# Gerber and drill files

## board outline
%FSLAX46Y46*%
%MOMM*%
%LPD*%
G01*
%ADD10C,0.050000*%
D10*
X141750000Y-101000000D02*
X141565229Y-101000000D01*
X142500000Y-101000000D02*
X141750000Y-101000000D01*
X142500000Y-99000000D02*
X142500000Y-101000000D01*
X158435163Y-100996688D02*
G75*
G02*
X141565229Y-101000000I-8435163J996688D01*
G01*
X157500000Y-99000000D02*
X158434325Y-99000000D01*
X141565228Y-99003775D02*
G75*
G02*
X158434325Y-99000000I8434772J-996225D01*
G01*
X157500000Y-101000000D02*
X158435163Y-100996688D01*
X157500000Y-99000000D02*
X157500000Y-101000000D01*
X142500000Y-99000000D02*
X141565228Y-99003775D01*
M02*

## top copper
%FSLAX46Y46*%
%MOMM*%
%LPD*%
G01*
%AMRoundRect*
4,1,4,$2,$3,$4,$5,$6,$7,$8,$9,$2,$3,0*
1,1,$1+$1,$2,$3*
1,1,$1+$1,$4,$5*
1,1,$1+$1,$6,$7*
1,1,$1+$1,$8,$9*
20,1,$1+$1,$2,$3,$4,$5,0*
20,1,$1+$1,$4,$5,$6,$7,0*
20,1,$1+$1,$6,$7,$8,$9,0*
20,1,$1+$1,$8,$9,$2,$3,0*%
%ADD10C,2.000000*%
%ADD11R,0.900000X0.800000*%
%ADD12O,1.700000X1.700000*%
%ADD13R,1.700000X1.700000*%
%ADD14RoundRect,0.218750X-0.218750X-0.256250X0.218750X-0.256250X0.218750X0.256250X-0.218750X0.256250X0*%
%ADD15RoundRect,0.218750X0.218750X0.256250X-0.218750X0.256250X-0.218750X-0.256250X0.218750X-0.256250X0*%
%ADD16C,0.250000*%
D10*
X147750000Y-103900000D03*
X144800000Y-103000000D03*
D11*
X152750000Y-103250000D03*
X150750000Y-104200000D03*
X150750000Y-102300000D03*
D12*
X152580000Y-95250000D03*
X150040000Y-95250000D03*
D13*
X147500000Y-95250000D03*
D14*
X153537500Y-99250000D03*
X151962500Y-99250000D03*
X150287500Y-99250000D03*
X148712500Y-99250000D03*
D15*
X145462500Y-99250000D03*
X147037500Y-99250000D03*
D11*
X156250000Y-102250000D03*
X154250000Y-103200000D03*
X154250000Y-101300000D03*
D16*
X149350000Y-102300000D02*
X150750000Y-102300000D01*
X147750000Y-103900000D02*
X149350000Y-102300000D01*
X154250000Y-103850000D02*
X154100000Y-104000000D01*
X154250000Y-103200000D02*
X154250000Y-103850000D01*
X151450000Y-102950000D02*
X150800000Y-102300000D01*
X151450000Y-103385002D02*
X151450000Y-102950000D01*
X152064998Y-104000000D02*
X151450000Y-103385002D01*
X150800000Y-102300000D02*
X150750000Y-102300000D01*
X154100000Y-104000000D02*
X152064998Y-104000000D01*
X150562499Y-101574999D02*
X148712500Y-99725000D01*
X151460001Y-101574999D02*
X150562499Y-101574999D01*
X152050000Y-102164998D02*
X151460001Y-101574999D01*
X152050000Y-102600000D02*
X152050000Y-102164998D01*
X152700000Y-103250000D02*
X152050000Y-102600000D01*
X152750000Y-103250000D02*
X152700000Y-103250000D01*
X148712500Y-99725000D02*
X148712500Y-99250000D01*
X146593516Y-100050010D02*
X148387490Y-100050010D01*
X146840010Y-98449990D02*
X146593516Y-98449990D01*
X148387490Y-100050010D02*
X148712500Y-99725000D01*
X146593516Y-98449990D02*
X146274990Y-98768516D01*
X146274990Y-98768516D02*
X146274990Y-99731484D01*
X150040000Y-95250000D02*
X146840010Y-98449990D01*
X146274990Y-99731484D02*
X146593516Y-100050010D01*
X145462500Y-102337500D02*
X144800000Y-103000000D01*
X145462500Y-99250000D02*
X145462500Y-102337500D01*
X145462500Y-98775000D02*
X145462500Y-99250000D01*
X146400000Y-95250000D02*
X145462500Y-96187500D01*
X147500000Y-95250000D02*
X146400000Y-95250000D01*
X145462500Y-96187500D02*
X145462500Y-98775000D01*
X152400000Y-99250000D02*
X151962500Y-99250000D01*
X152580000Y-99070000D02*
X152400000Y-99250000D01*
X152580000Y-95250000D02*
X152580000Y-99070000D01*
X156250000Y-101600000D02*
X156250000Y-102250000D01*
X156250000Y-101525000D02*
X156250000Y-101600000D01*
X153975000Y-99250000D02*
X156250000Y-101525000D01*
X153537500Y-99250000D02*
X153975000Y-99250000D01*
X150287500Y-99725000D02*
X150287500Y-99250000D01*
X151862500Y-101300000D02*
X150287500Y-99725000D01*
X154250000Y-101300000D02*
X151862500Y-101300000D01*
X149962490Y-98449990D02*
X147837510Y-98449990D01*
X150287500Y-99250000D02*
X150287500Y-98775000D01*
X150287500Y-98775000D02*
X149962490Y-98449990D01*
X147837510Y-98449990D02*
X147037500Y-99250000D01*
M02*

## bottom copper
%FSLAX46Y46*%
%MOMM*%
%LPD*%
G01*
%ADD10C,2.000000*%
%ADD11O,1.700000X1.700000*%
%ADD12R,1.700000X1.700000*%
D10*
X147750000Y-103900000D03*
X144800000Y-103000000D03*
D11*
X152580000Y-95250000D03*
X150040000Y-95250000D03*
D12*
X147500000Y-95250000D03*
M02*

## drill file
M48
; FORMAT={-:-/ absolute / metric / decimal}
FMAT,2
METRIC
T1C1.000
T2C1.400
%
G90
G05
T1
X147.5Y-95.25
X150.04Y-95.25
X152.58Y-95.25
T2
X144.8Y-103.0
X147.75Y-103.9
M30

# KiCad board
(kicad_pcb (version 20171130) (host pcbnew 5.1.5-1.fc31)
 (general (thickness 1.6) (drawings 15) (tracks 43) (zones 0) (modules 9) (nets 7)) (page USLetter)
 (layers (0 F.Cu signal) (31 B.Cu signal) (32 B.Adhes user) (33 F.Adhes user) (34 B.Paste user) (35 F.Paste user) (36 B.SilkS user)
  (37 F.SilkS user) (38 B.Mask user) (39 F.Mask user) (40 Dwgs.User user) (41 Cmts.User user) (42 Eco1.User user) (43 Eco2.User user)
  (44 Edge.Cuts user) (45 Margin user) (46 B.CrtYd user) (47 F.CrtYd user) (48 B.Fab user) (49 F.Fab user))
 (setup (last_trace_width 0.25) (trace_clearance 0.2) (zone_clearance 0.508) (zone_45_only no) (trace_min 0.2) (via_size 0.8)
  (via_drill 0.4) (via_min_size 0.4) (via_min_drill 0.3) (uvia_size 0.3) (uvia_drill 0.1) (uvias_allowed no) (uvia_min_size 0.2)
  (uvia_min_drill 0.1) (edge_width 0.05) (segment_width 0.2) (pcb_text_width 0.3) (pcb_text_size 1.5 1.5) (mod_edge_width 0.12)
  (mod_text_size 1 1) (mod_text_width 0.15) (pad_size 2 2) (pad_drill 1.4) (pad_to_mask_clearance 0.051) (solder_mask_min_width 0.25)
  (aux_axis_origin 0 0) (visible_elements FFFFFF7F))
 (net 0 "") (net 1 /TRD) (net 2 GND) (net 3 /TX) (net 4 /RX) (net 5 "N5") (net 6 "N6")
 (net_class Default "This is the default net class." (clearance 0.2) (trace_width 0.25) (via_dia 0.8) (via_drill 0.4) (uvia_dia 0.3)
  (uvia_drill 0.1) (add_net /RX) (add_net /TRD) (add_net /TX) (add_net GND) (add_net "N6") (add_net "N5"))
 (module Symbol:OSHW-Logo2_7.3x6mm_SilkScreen (layer B.Cu) (at 152.5 99.75 180)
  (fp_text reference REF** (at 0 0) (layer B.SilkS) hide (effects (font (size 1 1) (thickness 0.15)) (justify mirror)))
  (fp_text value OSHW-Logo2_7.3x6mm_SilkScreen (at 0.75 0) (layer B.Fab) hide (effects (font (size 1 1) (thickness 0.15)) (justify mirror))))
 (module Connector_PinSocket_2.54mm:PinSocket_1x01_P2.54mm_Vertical (layer B.Cu) (at 147.75 103.9)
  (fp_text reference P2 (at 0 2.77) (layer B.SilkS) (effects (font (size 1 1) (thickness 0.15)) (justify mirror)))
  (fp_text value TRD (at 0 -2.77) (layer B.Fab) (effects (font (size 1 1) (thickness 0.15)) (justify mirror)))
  (pad 1 thru_hole circle (at 0 0) (size 2 2) (drill 1.4) (layers *.Cu *.Mask) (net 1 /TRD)))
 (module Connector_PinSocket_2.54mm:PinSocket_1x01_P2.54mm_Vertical (layer B.Cu) (at 144.8 103)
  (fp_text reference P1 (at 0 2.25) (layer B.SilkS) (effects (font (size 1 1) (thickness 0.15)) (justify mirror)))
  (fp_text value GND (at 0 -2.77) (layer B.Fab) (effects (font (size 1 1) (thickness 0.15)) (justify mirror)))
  (pad 1 thru_hole circle (at 0 0) (size 2 2) (drill 1.4) (layers *.Cu *.Mask) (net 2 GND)))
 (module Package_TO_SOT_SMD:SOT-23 (layer F.Cu) (at 151.75 103.25)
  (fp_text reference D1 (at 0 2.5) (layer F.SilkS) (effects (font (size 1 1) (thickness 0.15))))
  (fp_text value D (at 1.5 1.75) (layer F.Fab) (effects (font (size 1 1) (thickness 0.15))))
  (pad 3 smd rect (at 1 0) (size 0.9 0.8) (layers F.Cu F.Paste F.Mask) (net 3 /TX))
  (pad 2 smd rect (at -1 0.95) (size 0.9 0.8) (layers F.Cu F.Paste F.Mask))
  (pad 1 smd rect (at -1 -0.95) (size 0.9 0.8) (layers F.Cu F.Paste F.Mask) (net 1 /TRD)))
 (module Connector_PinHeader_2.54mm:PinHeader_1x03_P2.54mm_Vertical (layer F.Cu) (at 147.5 95.25 90)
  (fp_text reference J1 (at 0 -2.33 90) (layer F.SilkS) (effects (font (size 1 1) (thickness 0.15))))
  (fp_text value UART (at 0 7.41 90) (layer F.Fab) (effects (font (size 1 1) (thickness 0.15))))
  (pad 3 thru_hole oval (at 0 5.08 90) (size 1.7 1.7) (drill 1) (layers *.Cu *.Mask) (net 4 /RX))
  (pad 2 thru_hole oval (at 0 2.54 90) (size 1.7 1.7) (drill 1) (layers *.Cu *.Mask) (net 3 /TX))
  (pad 1 thru_hole rect (at 0 0 90) (size 1.7 1.7) (drill 1) (layers *.Cu *.Mask) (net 2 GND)))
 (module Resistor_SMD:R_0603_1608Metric (layer F.Cu) (at 152.75 99.25)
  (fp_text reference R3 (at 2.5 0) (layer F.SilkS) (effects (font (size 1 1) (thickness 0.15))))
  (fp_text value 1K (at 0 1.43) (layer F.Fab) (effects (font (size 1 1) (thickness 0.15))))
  (pad 2 smd roundrect (at 0.7875 0) (size 0.875 0.95) (layers F.Cu F.Paste F.Mask) (roundrect_rratio 0.25) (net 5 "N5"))
  (pad 1 smd roundrect (at -0.7875 0) (size 0.875 0.95) (layers F.Cu F.Paste F.Mask) (roundrect_rratio 0.25) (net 4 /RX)))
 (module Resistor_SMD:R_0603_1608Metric (layer F.Cu) (at 149.5 99.25)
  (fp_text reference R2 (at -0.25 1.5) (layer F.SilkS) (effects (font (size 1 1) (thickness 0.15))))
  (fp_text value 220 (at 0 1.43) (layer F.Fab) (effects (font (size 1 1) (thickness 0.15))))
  (pad 2 smd roundrect (at 0.7875 0) (size 0.875 0.95) (layers F.Cu F.Paste F.Mask) (roundrect_rratio 0.25) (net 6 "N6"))
  (pad 1 smd roundrect (at -0.7875 0) (size 0.875 0.95) (layers F.Cu F.Paste F.Mask) (roundrect_rratio 0.25) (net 3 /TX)))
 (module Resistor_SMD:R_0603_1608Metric (layer F.Cu) (at 146.25 99.25 180)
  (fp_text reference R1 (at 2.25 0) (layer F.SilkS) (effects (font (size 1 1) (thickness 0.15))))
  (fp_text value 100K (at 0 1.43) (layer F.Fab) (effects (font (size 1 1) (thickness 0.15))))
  (pad 2 smd roundrect (at 0.7875 0 180) (size 0.875 0.95) (layers F.Cu F.Paste F.Mask) (roundrect_rratio 0.25) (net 2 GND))
  (pad 1 smd roundrect (at -0.7875 0 180) (size 0.875 0.95) (layers F.Cu F.Paste F.Mask) (roundrect_rratio 0.25) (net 6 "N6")))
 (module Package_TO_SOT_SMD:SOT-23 (layer F.Cu) (at 155.25 102.25)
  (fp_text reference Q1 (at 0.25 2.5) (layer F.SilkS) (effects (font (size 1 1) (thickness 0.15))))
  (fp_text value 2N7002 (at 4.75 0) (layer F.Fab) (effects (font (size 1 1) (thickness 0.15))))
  (pad 3 smd rect (at 1 0) (size 0.9 0.8) (layers F.Cu F.Paste F.Mask) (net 5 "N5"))
  (pad 2 smd rect (at -1 0.95) (size 0.9 0.8) (layers F.Cu F.Paste F.Mask) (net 1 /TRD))
  (pad 1 smd rect (at -1 -0.95) (size 0.9 0.8) (layers F.Cu F.Paste F.Mask) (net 6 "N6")))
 (gr_line (start 141.75 101) (end 141.565229 101) (layer Edge.Cuts) (width 0.05))
 (gr_line (start 142.5 101) (end 141.75 101) (layer Edge.Cuts) (width 0.05))
 (gr_line (start 142.5 99) (end 142.5 101) (layer Edge.Cuts) (width 0.05))
 (gr_arc (start 150 100) (end 141.565229 101) (angle -166.5) (layer Edge.Cuts) (width 0.05))
 (gr_line (start 157.5 99) (end 158.434325 99) (layer Edge.Cuts) (width 0.05))
 (gr_arc (start 150 100) (end 158.434325 99) (angle -166.5024402) (layer Edge.Cuts) (width 0.05))
 (gr_line (start 157.5 101) (end 158.435163 100.996688) (layer Edge.Cuts) (width 0.05))
 (gr_line (start 157.5 99) (end 157.5 101) (layer Edge.Cuts) (width 0.05))
 (gr_line (start 142.5 99) (end 141.565228 99.003775) (layer Edge.Cuts) (width 0.05))
 (segment (start 149.35 102.3) (end 150.75 102.3) (width 0.25) (layer F.Cu) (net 1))
 (segment (start 147.75 103.9) (end 149.35 102.3) (width 0.25) (layer F.Cu) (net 1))
 (segment (start 154.25 103.85) (end 154.1 104) (width 0.25) (layer F.Cu) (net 1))
 (segment (start 154.25 103.2) (end 154.25 103.85) (width 0.25) (layer F.Cu) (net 1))
 (segment (start 151.45 102.95) (end 150.8 102.3) (width 0.25) (layer F.Cu) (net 1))
 (segment (start 151.45 103.385002) (end 151.45 102.95) (width 0.25) (layer F.Cu) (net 1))
 (segment (start 152.064998 104) (end 151.45 103.385002) (width 0.25) (layer F.Cu) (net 1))
 (segment (start 150.8 102.3) (end 150.75 102.3) (width 0.25) (layer F.Cu) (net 1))
 (segment (start 154.1 104) (end 152.064998 104) (width 0.25) (layer F.Cu) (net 1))
 (segment (start 150.562499 101.574999) (end 148.7125 99.725) (width 0.25) (layer F.Cu) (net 3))
 (segment (start 151.460001 101.574999) (end 150.562499 101.574999) (width 0.25) (layer F.Cu) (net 3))
 (segment (start 152.05 102.164998) (end 151.460001 101.574999) (width 0.25) (layer F.Cu) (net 3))
 (segment (start 152.05 102.6) (end 152.05 102.164998) (width 0.25) (layer F.Cu) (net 3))
 (segment (start 152.7 103.25) (end 152.05 102.6) (width 0.25) (layer F.Cu) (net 3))
 (segment (start 152.75 103.25) (end 152.7 103.25) (width 0.25) (layer F.Cu) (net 3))
 (segment (start 148.7125 99.725) (end 148.7125 99.25) (width 0.25) (layer F.Cu) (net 3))
 (segment (start 146.593516 100.05001) (end 148.38749 100.05001) (width 0.25) (layer F.Cu) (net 3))
 (segment (start 146.84001 98.44999) (end 146.593516 98.44999) (width 0.25) (layer F.Cu) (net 3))
 (segment (start 148.38749 100.05001) (end 148.7125 99.725) (width 0.25) (layer F.Cu) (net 3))
 (segment (start 146.593516 98.44999) (end 146.27499 98.768516) (width 0.25) (layer F.Cu) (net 3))
 (segment (start 146.27499 98.768516) (end 146.27499 99.731484) (width 0.25) (layer F.Cu) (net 3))
 (segment (start 150.04 95.25) (end 146.84001 98.44999) (width 0.25) (layer F.Cu) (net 3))
 (segment (start 146.27499 99.731484) (end 146.593516 100.05001) (width 0.25) (layer F.Cu) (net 3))
 (segment (start 145.4625 102.3375) (end 144.8 103) (width 0.25) (layer F.Cu) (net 2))
 (segment (start 145.4625 99.25) (end 145.4625 102.3375) (width 0.25) (layer F.Cu) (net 2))
 (segment (start 145.4625 98.775) (end 145.4625 99.25) (width 0.25) (layer F.Cu) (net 2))
 (segment (start 146.4 95.25) (end 145.4625 96.1875) (width 0.25) (layer F.Cu) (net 2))
 (segment (start 147.5 95.25) (end 146.4 95.25) (width 0.25) (layer F.Cu) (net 2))
 (segment (start 145.4625 96.1875) (end 145.4625 98.775) (width 0.25) (layer F.Cu) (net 2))
 (segment (start 152.4 99.25) (end 151.9625 99.25) (width 0.25) (layer F.Cu) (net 4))
 (segment (start 152.58 99.07) (end 152.4 99.25) (width 0.25) (layer F.Cu) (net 4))
 (segment (start 152.58 95.25) (end 152.58 99.07) (width 0.25) (layer F.Cu) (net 4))
 (segment (start 156.25 101.6) (end 156.25 102.25) (width 0.25) (layer F.Cu) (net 5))
 (segment (start 156.25 101.525) (end 156.25 101.6) (width 0.25) (layer F.Cu) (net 5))
 (segment (start 153.975 99.25) (end 156.25 101.525) (width 0.25) (layer F.Cu) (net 5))
 (segment (start 153.5375 99.25) (end 153.975 99.25) (width 0.25) (layer F.Cu) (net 5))
 (segment (start 150.2875 99.725) (end 150.2875 99.25) (width 0.25) (layer F.Cu) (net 6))
 (segment (start 151.8625 101.3) (end 150.2875 99.725) (width 0.25) (layer F.Cu) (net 6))
 (segment (start 154.25 101.3) (end 151.8625 101.3) (width 0.25) (layer F.Cu) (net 6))
 (segment (start 149.96249 98.44999) (end 147.83751 98.44999) (width 0.25) (layer F.Cu) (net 6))
 (segment (start 150.2875 99.25) (end 150.2875 98.775) (width 0.25) (layer F.Cu) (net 6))
 (segment (start 150.2875 98.775) (end 149.96249 98.44999) (width 0.25) (layer F.Cu) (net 6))
 (segment (start 147.83751 98.44999) (end 147.0375 99.25) (width 0.25) (layer F.Cu) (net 6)))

